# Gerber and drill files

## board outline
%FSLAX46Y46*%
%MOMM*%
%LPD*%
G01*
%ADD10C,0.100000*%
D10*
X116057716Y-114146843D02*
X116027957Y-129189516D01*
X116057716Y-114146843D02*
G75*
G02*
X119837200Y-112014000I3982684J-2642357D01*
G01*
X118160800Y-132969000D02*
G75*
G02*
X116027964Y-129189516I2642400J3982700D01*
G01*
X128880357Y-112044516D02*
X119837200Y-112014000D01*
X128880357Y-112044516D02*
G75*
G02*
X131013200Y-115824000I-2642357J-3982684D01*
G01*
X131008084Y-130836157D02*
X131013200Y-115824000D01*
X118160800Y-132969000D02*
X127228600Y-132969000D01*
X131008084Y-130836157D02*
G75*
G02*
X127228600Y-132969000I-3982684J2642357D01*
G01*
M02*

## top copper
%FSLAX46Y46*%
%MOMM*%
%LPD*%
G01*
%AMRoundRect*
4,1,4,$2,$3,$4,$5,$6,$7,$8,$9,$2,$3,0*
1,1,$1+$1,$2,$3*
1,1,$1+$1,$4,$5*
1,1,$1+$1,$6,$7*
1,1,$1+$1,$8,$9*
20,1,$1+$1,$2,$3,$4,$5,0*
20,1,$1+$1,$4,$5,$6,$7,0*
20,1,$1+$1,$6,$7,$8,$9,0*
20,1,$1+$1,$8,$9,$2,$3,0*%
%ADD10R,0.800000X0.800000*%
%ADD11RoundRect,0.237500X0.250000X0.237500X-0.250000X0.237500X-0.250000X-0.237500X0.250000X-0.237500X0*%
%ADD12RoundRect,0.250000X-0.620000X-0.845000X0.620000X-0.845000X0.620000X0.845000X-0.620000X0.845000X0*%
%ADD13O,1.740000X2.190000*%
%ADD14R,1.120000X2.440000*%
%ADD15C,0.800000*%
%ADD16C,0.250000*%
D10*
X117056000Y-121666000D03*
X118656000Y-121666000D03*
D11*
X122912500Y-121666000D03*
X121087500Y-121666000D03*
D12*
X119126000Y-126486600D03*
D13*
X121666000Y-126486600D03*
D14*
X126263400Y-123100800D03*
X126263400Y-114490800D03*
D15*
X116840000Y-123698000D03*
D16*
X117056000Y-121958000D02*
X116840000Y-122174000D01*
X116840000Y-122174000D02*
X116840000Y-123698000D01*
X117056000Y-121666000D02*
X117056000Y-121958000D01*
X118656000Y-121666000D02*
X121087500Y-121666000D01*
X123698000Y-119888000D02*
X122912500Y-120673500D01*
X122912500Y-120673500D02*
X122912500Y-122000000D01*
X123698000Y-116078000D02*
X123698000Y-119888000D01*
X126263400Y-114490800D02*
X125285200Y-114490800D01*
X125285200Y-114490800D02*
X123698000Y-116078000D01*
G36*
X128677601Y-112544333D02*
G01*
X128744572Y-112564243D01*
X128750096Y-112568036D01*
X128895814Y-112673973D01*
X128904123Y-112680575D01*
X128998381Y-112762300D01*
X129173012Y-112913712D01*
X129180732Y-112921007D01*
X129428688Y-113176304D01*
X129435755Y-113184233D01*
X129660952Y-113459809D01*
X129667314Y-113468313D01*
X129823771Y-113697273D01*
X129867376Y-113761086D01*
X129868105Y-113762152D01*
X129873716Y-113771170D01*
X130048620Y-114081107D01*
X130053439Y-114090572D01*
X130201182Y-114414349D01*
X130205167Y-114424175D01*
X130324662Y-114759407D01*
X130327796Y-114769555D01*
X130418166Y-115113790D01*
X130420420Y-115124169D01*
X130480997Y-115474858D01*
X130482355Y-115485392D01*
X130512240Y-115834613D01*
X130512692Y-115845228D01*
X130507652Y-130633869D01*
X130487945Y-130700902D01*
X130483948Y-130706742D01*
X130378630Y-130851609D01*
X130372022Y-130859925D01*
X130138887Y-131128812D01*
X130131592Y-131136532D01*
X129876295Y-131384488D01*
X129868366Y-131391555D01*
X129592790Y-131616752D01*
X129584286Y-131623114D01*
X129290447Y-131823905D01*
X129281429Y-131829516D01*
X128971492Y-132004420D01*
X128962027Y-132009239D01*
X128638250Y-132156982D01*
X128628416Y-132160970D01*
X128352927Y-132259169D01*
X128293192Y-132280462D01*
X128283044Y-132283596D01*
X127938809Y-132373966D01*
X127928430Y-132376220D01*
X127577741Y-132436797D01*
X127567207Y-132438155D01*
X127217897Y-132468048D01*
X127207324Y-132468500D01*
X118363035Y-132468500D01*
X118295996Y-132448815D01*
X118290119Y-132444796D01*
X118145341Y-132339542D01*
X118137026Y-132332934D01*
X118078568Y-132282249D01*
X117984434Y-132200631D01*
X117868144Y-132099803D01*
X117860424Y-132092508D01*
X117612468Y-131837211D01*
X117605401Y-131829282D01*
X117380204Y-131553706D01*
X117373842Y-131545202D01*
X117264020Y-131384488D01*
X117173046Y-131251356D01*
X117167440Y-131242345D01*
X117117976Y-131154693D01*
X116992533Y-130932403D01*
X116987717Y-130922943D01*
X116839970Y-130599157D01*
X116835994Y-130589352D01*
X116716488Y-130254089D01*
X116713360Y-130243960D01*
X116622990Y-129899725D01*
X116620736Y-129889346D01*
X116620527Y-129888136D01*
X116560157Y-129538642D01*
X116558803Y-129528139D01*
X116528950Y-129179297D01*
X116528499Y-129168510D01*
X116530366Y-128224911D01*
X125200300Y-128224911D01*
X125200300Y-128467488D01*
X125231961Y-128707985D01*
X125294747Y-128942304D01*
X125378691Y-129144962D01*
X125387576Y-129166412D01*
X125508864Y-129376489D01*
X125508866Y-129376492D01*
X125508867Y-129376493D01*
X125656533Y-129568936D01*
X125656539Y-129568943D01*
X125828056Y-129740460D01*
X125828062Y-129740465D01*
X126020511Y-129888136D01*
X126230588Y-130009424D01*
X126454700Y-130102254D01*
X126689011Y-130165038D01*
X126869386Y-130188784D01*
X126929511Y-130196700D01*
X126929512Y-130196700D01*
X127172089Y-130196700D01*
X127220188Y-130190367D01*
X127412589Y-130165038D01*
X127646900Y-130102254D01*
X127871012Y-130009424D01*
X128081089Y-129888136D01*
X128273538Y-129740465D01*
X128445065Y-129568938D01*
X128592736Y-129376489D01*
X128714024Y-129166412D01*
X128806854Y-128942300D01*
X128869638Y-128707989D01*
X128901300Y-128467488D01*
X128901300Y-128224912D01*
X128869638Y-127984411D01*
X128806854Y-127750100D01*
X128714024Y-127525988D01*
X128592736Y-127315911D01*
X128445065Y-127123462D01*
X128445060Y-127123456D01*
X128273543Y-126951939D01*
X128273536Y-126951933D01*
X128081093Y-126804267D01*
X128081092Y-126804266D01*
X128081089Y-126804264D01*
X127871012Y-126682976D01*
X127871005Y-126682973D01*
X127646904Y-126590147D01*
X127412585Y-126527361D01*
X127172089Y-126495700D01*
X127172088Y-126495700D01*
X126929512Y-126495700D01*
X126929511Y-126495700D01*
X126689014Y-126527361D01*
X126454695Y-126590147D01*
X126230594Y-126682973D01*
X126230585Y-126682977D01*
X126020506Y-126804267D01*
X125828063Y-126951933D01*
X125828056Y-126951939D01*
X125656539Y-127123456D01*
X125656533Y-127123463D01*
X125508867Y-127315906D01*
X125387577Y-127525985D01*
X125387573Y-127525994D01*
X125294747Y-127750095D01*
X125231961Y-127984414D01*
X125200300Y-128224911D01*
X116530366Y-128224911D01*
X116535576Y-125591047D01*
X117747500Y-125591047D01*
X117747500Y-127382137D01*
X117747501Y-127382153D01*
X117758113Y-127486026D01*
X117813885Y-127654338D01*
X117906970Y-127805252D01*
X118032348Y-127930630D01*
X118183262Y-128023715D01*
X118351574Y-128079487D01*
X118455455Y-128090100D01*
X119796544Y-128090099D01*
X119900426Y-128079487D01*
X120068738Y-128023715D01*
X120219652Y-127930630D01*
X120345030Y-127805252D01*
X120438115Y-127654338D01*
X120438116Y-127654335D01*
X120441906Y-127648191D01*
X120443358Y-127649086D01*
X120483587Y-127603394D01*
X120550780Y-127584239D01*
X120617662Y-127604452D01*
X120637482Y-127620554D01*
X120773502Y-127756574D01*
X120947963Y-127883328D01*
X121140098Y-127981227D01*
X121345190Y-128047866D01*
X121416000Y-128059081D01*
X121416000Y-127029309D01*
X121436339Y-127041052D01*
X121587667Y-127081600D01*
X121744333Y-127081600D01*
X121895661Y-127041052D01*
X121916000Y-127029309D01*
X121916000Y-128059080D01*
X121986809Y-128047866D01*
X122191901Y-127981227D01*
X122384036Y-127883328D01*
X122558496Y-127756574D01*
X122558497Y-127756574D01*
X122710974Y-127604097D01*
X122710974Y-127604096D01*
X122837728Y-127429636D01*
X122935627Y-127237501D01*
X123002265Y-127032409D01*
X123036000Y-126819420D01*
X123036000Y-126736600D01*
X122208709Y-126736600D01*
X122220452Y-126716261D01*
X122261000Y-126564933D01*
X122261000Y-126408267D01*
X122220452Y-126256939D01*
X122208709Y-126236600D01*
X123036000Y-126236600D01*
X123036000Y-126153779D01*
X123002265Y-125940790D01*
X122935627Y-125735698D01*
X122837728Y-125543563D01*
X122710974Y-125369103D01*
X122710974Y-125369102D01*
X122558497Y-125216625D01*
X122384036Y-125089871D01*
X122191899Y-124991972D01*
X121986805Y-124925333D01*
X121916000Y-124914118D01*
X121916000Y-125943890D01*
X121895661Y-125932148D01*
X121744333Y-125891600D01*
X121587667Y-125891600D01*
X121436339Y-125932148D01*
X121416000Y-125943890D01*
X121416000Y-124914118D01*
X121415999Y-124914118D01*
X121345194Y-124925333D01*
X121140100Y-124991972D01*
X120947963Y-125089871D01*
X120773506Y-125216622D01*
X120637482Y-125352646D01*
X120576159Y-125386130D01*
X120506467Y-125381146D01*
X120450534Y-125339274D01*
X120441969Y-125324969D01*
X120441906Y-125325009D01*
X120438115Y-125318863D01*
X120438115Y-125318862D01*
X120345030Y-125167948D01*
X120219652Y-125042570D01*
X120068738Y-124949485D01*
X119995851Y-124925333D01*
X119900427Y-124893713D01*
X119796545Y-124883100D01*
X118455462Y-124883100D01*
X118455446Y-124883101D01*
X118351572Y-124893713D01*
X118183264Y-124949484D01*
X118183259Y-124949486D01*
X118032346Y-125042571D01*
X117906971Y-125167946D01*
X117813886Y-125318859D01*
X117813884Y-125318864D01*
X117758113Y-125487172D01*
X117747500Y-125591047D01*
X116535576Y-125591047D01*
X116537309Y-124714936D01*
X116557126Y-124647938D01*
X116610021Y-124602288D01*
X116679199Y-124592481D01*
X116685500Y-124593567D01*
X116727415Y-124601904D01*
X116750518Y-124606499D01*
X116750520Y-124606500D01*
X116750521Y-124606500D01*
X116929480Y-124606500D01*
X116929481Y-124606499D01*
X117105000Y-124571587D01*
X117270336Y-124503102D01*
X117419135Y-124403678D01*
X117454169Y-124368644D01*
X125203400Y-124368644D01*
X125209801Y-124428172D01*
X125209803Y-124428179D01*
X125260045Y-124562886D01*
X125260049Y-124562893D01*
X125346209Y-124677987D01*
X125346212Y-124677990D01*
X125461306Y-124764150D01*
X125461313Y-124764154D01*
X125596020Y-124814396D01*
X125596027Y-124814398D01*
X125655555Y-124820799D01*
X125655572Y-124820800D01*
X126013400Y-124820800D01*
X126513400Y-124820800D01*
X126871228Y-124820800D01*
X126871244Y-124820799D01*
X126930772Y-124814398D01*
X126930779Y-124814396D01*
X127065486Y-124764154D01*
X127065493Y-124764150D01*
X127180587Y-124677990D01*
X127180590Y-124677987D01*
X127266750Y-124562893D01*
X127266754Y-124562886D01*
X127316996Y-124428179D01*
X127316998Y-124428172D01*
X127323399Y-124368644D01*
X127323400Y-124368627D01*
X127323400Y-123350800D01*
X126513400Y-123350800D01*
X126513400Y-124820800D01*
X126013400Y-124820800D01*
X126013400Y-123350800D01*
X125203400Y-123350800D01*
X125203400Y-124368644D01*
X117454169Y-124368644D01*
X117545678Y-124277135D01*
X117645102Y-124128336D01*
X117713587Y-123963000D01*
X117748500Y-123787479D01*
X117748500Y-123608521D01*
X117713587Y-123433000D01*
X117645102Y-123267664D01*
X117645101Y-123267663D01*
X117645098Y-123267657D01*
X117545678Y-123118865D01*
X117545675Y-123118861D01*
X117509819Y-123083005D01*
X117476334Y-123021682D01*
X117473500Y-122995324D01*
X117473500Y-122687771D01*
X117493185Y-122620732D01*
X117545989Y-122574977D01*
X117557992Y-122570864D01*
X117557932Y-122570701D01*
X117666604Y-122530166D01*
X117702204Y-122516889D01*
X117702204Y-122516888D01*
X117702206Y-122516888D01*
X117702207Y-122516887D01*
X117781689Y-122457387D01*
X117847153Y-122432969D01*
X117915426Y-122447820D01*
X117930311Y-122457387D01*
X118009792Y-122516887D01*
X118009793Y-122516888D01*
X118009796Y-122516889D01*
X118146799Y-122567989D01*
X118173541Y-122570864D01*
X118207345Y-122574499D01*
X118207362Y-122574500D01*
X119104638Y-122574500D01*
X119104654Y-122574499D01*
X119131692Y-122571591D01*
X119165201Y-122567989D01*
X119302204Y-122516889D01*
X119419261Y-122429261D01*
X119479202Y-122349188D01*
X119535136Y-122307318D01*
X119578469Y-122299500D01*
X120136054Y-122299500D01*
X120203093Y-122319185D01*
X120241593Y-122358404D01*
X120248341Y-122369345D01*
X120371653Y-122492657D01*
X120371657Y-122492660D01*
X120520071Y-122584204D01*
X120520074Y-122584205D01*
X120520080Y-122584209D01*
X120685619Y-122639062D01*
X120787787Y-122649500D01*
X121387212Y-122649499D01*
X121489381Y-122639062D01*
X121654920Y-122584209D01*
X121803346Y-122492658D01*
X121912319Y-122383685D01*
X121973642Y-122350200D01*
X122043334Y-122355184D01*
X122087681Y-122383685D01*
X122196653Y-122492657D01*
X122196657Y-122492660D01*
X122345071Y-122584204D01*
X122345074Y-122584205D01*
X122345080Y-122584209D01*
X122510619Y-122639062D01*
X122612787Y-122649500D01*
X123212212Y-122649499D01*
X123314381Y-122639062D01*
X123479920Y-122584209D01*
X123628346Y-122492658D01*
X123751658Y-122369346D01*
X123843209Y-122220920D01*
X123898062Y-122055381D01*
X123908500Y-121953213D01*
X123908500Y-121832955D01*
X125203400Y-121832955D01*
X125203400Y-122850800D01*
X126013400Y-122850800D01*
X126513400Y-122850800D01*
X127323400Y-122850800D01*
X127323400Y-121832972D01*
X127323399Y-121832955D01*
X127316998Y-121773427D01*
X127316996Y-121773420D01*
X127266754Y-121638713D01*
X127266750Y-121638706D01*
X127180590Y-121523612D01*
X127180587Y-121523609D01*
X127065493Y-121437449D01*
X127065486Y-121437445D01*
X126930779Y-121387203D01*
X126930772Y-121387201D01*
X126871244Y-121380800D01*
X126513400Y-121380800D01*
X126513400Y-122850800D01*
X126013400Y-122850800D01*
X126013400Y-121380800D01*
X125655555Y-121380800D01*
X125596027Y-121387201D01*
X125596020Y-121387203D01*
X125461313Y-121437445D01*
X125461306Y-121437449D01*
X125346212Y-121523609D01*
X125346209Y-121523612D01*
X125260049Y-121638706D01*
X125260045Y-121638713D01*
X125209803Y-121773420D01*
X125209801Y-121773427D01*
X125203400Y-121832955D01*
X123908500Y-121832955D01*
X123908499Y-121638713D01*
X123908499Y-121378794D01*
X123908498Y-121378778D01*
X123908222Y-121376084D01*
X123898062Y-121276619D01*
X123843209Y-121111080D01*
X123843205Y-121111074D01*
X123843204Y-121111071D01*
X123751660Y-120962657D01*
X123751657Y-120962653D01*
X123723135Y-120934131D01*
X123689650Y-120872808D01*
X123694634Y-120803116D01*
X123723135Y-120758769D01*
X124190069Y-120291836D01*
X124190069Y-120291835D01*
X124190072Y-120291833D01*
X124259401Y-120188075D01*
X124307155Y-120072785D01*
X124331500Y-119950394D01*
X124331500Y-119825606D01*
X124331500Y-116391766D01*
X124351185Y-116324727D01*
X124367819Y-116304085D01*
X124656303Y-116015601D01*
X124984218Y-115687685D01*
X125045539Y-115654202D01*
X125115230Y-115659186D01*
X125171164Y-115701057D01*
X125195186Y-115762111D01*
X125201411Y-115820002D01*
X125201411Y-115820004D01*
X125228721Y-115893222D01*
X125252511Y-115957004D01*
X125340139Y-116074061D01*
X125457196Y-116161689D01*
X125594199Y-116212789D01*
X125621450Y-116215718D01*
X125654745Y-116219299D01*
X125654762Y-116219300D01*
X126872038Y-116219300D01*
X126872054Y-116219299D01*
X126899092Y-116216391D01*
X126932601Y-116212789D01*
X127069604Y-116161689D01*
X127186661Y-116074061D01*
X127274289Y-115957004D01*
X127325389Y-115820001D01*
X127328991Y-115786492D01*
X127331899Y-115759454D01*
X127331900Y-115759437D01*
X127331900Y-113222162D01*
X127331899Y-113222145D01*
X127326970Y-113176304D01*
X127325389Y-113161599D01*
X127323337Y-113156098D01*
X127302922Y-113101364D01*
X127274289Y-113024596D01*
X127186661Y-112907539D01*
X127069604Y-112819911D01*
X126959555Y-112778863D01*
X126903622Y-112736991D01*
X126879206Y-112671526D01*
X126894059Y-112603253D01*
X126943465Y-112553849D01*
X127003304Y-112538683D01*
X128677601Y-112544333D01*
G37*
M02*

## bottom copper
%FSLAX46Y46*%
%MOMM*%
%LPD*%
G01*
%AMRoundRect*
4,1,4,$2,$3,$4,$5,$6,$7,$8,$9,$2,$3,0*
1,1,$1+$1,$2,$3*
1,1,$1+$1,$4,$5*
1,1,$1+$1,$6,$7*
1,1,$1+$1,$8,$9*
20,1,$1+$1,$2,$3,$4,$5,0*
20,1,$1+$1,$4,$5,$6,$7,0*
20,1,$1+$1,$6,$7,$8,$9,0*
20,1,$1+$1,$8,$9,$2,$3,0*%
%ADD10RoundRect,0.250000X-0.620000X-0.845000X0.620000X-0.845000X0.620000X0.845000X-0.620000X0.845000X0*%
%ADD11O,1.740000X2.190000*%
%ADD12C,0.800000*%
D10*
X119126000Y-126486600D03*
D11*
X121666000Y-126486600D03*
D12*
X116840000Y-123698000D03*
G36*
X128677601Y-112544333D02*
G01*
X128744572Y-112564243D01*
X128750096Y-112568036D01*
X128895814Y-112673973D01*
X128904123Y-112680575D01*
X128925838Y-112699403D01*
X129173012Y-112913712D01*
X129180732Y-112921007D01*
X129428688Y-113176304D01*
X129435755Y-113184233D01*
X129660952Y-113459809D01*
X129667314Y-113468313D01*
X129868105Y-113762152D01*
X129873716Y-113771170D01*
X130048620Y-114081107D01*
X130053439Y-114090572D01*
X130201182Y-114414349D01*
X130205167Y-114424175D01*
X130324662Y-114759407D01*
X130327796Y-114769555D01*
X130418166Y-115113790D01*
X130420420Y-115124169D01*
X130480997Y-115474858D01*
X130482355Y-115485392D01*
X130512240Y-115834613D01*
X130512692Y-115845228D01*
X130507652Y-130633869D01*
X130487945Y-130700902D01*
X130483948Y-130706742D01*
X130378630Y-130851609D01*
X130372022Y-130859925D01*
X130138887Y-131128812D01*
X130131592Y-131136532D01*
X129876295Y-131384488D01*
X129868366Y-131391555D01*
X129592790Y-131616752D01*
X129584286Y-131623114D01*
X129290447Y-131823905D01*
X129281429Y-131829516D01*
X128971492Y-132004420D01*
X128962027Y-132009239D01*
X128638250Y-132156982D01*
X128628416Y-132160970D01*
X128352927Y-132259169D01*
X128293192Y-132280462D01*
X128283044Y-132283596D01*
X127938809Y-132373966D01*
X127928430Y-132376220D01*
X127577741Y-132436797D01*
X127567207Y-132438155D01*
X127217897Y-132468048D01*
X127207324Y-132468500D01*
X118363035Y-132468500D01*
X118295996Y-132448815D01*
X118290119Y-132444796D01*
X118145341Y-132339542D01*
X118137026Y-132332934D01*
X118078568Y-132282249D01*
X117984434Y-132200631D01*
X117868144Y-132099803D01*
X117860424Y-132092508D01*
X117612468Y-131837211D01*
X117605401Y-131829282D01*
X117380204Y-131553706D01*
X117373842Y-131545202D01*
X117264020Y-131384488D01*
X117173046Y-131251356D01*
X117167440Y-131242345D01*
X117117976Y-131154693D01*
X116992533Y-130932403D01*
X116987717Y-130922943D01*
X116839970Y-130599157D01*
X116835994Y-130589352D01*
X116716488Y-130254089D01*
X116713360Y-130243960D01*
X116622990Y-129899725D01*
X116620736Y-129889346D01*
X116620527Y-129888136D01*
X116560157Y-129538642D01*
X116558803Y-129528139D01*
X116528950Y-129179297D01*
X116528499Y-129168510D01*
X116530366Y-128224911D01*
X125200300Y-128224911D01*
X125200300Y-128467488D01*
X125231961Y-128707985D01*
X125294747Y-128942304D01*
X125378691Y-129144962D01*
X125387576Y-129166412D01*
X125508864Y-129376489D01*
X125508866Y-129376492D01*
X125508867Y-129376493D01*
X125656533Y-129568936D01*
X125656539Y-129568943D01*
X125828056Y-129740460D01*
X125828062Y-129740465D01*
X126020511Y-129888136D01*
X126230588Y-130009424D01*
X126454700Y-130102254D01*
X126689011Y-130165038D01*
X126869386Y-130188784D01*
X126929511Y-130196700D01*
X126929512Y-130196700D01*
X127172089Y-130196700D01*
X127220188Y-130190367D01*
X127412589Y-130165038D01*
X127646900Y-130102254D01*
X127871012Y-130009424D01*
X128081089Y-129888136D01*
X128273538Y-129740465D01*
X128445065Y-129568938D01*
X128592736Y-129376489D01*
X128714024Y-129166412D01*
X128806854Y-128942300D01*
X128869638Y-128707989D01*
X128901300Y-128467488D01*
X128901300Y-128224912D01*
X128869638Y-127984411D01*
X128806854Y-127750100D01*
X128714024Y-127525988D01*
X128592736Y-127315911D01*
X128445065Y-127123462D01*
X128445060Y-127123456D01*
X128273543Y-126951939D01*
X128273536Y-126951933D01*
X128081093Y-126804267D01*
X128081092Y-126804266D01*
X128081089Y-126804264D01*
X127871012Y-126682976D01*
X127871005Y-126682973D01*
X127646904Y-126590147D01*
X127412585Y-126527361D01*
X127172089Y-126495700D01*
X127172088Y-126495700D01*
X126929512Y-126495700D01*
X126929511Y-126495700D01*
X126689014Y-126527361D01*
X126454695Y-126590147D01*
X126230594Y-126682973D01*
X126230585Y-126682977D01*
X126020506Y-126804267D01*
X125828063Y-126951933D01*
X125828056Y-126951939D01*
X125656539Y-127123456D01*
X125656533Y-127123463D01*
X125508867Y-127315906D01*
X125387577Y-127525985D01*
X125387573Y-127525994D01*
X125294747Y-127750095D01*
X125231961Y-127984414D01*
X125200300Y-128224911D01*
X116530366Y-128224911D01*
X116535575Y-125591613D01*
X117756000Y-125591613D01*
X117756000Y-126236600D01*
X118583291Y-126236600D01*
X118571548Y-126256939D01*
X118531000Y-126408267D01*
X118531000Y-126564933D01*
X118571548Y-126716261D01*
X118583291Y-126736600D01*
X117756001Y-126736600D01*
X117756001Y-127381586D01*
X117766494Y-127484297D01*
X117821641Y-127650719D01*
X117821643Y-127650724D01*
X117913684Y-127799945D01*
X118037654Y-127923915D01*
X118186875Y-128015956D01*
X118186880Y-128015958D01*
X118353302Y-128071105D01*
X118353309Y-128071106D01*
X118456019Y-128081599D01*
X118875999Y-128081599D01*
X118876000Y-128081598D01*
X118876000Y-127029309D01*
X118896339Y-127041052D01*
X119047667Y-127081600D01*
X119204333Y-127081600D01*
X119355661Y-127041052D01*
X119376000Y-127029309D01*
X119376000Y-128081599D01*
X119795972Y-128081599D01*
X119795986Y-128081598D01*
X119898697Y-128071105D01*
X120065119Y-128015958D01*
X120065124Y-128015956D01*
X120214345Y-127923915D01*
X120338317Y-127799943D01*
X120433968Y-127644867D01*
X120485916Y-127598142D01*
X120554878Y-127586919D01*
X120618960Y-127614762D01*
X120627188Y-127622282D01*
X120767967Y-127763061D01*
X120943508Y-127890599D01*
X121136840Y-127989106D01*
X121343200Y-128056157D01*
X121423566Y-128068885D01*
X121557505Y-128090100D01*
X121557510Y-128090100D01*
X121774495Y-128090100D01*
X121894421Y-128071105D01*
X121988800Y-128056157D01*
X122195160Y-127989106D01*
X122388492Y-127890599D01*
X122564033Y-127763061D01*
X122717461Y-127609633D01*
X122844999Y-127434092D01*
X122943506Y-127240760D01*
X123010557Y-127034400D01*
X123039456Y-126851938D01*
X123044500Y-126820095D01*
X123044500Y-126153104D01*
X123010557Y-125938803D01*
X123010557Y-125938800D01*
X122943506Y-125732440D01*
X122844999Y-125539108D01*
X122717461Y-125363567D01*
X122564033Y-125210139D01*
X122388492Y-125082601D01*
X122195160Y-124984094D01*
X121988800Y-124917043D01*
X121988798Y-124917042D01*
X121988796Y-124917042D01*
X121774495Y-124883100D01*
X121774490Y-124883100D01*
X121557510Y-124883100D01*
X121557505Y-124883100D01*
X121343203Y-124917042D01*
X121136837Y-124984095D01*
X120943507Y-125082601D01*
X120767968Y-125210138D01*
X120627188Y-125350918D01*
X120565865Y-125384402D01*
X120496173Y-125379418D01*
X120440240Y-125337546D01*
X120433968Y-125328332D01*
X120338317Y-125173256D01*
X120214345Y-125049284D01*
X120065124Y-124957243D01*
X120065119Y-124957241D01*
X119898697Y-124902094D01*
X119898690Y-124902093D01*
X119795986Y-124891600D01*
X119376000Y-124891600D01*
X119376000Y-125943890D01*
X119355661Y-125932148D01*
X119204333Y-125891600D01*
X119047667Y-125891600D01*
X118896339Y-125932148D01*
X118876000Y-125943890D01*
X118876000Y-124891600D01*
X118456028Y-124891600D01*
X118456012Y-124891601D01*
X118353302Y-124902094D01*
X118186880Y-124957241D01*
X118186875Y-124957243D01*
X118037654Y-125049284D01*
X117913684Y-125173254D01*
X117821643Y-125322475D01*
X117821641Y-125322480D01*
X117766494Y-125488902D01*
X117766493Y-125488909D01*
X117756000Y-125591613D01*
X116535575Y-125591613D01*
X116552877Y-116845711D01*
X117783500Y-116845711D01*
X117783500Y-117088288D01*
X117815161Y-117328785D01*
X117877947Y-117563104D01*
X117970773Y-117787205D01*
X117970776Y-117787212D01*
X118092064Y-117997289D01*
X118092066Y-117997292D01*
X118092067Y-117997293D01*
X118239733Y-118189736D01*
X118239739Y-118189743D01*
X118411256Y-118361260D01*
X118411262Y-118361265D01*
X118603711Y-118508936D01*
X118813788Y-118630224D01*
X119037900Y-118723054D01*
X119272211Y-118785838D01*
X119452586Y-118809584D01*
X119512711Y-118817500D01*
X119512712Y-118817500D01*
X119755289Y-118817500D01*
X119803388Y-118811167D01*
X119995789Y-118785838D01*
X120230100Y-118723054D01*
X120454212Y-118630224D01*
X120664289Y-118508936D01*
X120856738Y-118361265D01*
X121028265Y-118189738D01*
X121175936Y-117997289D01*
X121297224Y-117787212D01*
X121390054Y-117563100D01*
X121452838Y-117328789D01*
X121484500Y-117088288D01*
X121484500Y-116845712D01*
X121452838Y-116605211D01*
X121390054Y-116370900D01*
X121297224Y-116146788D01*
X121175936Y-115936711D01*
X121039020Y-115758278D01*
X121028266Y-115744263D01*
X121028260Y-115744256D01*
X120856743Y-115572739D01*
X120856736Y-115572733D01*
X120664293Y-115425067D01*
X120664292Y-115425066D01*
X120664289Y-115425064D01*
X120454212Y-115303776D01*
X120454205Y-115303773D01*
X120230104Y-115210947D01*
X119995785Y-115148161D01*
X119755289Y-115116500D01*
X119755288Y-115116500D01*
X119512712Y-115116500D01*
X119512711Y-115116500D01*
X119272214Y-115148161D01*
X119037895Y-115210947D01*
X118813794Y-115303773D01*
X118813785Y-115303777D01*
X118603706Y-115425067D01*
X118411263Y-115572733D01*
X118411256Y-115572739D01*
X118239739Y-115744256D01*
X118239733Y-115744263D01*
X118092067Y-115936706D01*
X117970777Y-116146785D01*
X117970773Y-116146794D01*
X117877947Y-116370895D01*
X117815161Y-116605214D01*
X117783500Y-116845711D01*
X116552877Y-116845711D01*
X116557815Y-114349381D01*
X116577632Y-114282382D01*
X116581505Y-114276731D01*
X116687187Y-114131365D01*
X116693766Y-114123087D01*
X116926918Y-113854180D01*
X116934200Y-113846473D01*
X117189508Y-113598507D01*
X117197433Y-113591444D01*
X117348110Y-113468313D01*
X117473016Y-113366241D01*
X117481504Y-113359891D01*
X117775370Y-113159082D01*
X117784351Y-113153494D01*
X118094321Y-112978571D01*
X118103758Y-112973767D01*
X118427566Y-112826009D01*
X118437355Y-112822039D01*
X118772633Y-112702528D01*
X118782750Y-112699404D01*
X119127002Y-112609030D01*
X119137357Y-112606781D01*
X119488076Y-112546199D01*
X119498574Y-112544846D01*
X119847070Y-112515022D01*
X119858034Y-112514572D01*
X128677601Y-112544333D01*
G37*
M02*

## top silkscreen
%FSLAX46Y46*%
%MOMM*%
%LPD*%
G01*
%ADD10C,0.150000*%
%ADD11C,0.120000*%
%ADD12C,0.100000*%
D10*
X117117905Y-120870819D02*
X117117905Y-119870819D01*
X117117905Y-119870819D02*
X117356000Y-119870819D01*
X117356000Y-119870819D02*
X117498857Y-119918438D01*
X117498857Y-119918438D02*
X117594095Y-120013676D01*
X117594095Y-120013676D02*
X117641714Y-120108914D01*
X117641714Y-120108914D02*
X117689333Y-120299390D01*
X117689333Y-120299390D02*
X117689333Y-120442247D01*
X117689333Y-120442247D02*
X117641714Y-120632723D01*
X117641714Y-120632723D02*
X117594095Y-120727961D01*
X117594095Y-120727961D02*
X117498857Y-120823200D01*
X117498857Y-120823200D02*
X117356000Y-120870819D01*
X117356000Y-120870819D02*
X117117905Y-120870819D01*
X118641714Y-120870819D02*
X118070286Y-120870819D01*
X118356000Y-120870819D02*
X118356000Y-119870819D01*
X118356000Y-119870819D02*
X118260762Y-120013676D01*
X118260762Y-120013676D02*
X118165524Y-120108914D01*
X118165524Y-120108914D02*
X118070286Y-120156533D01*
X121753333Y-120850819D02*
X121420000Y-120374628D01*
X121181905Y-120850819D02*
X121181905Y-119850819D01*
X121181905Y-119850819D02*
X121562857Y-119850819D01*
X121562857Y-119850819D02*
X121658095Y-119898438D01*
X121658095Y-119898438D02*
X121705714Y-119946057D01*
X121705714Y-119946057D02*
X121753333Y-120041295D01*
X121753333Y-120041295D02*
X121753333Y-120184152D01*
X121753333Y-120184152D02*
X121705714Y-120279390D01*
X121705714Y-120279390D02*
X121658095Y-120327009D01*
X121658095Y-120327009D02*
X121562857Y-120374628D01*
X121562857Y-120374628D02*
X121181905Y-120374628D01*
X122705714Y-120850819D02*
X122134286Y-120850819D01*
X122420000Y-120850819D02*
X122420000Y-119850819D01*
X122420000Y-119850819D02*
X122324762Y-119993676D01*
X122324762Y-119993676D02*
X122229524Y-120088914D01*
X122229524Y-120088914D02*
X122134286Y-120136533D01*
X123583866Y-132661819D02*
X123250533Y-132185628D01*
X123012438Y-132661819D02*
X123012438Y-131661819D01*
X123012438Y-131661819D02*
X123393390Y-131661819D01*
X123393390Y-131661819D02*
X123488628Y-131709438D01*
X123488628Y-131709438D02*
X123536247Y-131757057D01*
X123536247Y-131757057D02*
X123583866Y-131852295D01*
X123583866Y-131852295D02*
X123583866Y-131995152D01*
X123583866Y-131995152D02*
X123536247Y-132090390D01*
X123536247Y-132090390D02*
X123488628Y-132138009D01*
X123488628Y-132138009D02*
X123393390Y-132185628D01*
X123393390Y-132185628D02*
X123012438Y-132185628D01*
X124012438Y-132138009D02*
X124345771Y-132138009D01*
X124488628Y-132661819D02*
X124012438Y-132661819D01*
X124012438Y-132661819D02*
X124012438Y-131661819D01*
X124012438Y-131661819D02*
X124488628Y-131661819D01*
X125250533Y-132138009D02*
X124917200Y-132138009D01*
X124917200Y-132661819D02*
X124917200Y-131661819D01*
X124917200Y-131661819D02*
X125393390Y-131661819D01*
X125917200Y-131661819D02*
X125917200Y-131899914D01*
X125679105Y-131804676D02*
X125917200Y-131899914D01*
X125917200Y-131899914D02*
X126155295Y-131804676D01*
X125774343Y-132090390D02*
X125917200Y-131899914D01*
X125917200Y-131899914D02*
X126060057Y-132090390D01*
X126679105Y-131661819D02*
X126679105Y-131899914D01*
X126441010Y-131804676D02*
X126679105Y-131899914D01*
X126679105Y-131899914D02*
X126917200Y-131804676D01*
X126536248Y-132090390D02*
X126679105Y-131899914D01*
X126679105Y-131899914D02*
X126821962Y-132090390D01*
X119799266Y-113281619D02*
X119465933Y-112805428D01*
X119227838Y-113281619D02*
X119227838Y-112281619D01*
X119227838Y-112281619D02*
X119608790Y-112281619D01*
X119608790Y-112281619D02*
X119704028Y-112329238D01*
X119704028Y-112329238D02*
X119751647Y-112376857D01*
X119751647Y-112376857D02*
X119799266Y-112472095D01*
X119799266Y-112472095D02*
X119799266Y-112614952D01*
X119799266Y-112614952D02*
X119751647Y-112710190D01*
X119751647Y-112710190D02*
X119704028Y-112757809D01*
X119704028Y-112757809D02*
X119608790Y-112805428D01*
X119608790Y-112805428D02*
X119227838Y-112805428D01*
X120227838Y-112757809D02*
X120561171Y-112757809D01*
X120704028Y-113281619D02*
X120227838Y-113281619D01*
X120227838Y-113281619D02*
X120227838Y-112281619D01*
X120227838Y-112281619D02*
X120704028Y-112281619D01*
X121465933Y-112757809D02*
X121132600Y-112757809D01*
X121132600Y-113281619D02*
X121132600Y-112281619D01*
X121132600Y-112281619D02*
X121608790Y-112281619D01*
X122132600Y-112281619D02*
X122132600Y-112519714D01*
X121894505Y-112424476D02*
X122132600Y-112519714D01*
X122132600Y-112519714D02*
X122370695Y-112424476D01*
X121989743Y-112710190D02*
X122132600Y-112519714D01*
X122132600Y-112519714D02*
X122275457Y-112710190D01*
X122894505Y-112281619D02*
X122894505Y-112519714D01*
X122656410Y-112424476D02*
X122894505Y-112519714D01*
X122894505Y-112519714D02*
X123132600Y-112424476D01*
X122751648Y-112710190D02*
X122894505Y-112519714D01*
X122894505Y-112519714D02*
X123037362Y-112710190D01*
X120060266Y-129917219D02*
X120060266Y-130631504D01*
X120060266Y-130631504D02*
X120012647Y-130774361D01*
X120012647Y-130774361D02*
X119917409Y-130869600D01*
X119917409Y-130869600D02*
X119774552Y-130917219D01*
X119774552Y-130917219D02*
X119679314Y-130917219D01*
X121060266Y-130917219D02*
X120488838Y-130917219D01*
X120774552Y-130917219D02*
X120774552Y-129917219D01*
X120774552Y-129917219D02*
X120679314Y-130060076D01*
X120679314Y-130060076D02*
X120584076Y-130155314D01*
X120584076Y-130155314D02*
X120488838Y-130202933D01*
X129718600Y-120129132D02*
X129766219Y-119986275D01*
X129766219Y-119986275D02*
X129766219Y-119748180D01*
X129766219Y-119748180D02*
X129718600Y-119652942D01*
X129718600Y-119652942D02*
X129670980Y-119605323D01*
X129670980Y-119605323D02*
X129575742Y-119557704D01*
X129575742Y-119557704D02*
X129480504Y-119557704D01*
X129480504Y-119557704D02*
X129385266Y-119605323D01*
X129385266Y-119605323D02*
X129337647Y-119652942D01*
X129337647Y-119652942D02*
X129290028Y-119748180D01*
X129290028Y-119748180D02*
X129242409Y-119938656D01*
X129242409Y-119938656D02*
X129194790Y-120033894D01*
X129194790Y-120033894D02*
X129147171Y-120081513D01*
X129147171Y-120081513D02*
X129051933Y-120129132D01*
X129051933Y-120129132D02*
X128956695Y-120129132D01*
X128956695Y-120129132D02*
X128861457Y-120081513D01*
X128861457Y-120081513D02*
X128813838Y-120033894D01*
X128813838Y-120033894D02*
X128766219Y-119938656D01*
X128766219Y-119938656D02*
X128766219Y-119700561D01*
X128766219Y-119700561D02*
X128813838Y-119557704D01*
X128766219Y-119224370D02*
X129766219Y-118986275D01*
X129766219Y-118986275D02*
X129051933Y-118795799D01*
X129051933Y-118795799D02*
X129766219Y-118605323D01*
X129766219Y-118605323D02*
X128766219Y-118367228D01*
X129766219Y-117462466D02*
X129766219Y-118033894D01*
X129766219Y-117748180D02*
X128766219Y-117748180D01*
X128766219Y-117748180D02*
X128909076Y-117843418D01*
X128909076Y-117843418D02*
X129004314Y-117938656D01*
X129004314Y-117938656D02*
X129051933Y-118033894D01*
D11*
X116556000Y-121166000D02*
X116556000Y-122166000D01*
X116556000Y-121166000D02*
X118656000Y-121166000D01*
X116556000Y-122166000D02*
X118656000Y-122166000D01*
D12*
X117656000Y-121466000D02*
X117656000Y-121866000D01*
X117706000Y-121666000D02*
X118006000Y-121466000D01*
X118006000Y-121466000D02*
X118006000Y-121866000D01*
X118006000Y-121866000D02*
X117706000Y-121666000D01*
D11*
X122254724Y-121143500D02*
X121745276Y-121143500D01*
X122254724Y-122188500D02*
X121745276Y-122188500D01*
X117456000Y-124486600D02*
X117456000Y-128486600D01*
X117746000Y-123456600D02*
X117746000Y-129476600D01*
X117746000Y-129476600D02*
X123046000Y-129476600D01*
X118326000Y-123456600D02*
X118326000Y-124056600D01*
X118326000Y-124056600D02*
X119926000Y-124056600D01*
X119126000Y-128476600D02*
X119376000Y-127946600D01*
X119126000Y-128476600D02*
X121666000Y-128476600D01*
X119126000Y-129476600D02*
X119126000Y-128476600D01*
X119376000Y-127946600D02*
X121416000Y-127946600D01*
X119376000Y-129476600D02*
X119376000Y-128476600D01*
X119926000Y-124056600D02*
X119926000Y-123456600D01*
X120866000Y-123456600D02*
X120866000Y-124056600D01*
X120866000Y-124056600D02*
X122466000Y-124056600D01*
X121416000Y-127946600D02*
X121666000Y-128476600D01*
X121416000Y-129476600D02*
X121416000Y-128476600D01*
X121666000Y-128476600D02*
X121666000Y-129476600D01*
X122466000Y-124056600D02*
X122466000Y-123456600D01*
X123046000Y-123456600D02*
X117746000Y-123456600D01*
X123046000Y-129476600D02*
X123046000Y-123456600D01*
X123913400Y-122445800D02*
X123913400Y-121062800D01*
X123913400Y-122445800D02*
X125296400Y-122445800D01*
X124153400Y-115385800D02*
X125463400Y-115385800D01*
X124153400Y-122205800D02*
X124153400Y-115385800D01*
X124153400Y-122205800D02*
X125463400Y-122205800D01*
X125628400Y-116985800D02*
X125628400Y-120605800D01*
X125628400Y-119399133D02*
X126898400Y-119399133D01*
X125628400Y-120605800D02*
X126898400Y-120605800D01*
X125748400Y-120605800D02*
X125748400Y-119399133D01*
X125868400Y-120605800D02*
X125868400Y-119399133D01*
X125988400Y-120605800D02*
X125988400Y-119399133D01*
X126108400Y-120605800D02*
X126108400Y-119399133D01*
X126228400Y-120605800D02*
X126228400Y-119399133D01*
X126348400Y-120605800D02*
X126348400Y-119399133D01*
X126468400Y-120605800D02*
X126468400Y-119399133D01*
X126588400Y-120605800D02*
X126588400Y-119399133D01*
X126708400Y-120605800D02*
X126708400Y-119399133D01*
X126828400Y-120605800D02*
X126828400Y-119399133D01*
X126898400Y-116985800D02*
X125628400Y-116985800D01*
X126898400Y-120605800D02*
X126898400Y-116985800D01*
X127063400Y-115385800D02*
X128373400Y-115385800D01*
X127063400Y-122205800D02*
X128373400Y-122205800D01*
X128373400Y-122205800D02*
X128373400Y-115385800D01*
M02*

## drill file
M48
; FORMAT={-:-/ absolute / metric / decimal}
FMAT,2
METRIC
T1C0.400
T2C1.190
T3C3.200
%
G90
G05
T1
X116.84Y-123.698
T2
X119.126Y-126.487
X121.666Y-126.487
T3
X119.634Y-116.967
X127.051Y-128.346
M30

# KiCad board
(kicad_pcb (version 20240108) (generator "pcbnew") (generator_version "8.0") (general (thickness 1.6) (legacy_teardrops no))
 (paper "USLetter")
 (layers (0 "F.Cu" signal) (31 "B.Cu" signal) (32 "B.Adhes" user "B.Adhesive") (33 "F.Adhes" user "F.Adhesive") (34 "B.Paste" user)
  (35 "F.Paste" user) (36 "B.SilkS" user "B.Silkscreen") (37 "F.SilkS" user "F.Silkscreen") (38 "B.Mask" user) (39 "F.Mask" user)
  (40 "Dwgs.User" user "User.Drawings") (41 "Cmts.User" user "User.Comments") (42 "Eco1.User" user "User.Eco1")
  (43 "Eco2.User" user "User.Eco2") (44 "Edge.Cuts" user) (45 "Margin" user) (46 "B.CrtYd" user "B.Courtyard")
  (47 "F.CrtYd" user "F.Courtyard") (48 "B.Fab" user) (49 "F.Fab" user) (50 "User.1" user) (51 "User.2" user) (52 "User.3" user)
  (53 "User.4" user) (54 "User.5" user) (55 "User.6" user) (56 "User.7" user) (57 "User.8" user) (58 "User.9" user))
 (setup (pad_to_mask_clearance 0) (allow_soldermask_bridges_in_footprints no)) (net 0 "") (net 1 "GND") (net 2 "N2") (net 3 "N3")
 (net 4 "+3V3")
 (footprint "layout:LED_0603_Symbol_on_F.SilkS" (layer "F.Cu") (at 117.856 121.666)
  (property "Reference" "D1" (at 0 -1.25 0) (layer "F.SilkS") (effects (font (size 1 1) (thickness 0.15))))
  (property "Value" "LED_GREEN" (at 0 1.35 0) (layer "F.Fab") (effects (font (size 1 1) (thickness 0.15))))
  (fp_line (start -1.3 -0.5) (end -1.3 0.5) (stroke (width 0.12) (type solid)) (layer "F.SilkS"))
  (fp_line (start -1.3 -0.5) (end 0.8 -0.5) (stroke (width 0.12) (type solid)) (layer "F.SilkS"))
  (fp_line (start -1.3 0.5) (end 0.8 0.5) (stroke (width 0.12) (type solid)) (layer "F.SilkS"))
  (fp_line (start -0.2 -0.2) (end -0.2 0.2) (stroke (width 0.1) (type solid)) (layer "F.SilkS"))
  (fp_line (start -0.15 0) (end 0.15 -0.2) (stroke (width 0.1) (type solid)) (layer "F.SilkS"))
  (fp_line (start 0.15 -0.2) (end 0.15 0.2) (stroke (width 0.1) (type solid)) (layer "F.SilkS"))
  (fp_line (start 0.15 0.2) (end -0.15 0) (stroke (width 0.1) (type solid)) (layer "F.SilkS"))
  (pad "1" smd rect (at -0.8 0 180) (size 0.8 0.8) (layers "F.Cu" "F.Paste" "F.Mask") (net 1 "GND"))
  (pad "2" smd rect (at 0.8 0 180) (size 0.8 0.8) (layers "F.Cu" "F.Paste" "F.Mask") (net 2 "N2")))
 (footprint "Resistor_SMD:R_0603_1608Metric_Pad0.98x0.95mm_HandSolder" (layer "F.Cu") (at 122 121.666 180)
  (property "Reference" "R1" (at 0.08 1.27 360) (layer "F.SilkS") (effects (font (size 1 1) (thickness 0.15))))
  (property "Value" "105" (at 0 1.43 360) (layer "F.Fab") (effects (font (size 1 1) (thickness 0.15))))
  (fp_line (start -0.254724 0.5225) (end 0.254724 0.5225) (stroke (width 0.12) (type solid)) (layer "F.SilkS"))
  (fp_line (start -0.254724 -0.5225) (end 0.254724 -0.5225) (stroke (width 0.12) (type solid)) (layer "F.SilkS"))
  (pad "1" smd roundrect (at -0.9125 0 180) (size 0.975 0.95) (layers "F.Cu" "F.Paste" "F.Mask") (roundrect_rratio 0.25) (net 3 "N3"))
  (pad "2" smd roundrect (at 0.9125 0 180) (size 0.975 0.95) (layers "F.Cu" "F.Paste" "F.Mask") (roundrect_rratio 0.25) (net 2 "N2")))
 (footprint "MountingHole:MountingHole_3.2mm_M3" (layer "F.Cu") (at 127.0508 128.3462)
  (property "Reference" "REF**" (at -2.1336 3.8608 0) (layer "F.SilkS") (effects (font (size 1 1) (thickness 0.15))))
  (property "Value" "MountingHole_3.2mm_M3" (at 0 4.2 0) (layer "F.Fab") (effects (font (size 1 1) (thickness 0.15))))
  (pad "" np_thru_hole circle (at 0 0) (size 3.2 3.2) (drill 3.2) (layers "*.Cu" "*.Mask")))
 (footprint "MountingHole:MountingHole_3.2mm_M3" (layer "F.Cu") (at 119.634 116.967)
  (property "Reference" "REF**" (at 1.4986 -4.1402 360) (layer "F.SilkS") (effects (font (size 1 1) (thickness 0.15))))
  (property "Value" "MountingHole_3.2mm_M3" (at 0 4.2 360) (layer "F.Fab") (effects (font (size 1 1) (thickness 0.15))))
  (pad "" np_thru_hole circle (at 0 0) (size 3.2 3.2) (drill 3.2) (layers "*.Cu" "*.Mask")))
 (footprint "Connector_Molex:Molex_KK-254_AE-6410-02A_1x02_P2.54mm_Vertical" (layer "F.Cu") (at 119.126 126.4866)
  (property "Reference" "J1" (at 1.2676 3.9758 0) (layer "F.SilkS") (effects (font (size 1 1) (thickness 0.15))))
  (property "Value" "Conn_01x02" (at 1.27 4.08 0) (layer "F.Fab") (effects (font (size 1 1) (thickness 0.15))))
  (fp_line (start -1.67 -2) (end -1.67 2) (stroke (width 0.12) (type solid)) (layer "F.SilkS"))
  (fp_line (start -1.38 -3.03) (end -1.38 2.99) (stroke (width 0.12) (type solid)) (layer "F.SilkS"))
  (fp_line (start -1.38 2.99) (end 3.92 2.99) (stroke (width 0.12) (type solid)) (layer "F.SilkS"))
  (fp_line (start -0.8 -3.03) (end -0.8 -2.43) (stroke (width 0.12) (type solid)) (layer "F.SilkS"))
  (fp_line (start -0.8 -2.43) (end 0.8 -2.43) (stroke (width 0.12) (type solid)) (layer "F.SilkS"))
  (fp_line (start 0 1.99) (end 0.25 1.46) (stroke (width 0.12) (type solid)) (layer "F.SilkS"))
  (fp_line (start 0 1.99) (end 2.54 1.99) (stroke (width 0.12) (type solid)) (layer "F.SilkS"))
  (fp_line (start 0 2.99) (end 0 1.99) (stroke (width 0.12) (type solid)) (layer "F.SilkS"))
  (fp_line (start 0.25 1.46) (end 2.29 1.46) (stroke (width 0.12) (type solid)) (layer "F.SilkS"))
  (fp_line (start 0.25 2.99) (end 0.25 1.99) (stroke (width 0.12) (type solid)) (layer "F.SilkS"))
  (fp_line (start 0.8 -2.43) (end 0.8 -3.03) (stroke (width 0.12) (type solid)) (layer "F.SilkS"))
  (fp_line (start 1.74 -3.03) (end 1.74 -2.43) (stroke (width 0.12) (type solid)) (layer "F.SilkS"))
  (fp_line (start 1.74 -2.43) (end 3.34 -2.43) (stroke (width 0.12) (type solid)) (layer "F.SilkS"))
  (fp_line (start 2.29 1.46) (end 2.54 1.99) (stroke (width 0.12) (type solid)) (layer "F.SilkS"))
  (fp_line (start 2.29 2.99) (end 2.29 1.99) (stroke (width 0.12) (type solid)) (layer "F.SilkS"))
  (fp_line (start 2.54 1.99) (end 2.54 2.99) (stroke (width 0.12) (type solid)) (layer "F.SilkS"))
  (fp_line (start 3.34 -2.43) (end 3.34 -3.03) (stroke (width 0.12) (type solid)) (layer "F.SilkS"))
  (fp_line (start 3.92 -3.03) (end -1.38 -3.03) (stroke (width 0.12) (type solid)) (layer "F.SilkS"))
  (fp_line (start 3.92 2.99) (end 3.92 -3.03) (stroke (width 0.12) (type solid)) (layer "F.SilkS"))
  (pad "1" thru_hole roundrect (at 0 0) (size 1.74 2.19) (drill 1.19) (layers "*.Cu" "*.Mask") (remove_unused_layers no)
   (roundrect_rratio 0.143678) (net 1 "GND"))
  (pad "2" thru_hole oval (at 2.54 0) (size 1.74 2.19) (drill 1.19) (layers "*.Cu" "*.Mask") (remove_unused_layers no) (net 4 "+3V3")))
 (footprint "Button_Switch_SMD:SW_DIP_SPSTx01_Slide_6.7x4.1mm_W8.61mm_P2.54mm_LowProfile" (layer "F.Cu") (at 126.2634 118.7958 90)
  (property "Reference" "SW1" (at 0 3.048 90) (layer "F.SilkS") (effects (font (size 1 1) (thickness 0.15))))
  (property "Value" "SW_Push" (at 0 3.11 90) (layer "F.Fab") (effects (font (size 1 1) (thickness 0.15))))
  (fp_line (start -3.65 -2.35) (end -2.267 -2.35) (stroke (width 0.12) (type solid)) (layer "F.SilkS"))
  (fp_line (start -3.65 -2.35) (end -3.65 -0.967) (stroke (width 0.12) (type solid)) (layer "F.SilkS"))
  (fp_line (start 3.41 -2.11) (end 3.41 -0.8) (stroke (width 0.12) (type solid)) (layer "F.SilkS"))
  (fp_line (start -3.41 -2.11) (end 3.41 -2.11) (stroke (width 0.12) (type solid)) (layer "F.SilkS"))
  (fp_line (start -3.41 -2.11) (end -3.41 -0.8) (stroke (width 0.12) (type solid)) (layer "F.SilkS"))
  (fp_line (start 1.81 -0.635) (end -1.81 -0.635) (stroke (width 0.12) (type solid)) (layer "F.SilkS"))
  (fp_line (start -0.603333 -0.635) (end -0.603333 0.635) (stroke (width 0.12) (type solid)) (layer "F.SilkS"))
  (fp_line (start -1.81 -0.635) (end -1.81 0.635) (stroke (width 0.12) (type solid)) (layer "F.SilkS"))
  (fp_line (start -1.81 -0.515) (end -0.603333 -0.515) (stroke (width 0.12) (type solid)) (layer "F.SilkS"))
  (fp_line (start -1.81 -0.395) (end -0.603333 -0.395) (stroke (width 0.12) (type solid)) (layer "F.SilkS"))
  (fp_line (start -1.81 -0.275) (end -0.603333 -0.275) (stroke (width 0.12) (type solid)) (layer "F.SilkS"))
  (fp_line (start -1.81 -0.155) (end -0.603333 -0.155) (stroke (width 0.12) (type solid)) (layer "F.SilkS"))
  (fp_line (start -1.81 -0.035) (end -0.603333 -0.035) (stroke (width 0.12) (type solid)) (layer "F.SilkS"))
  (fp_line (start -1.81 0.085) (end -0.603333 0.085) (stroke (width 0.12) (type solid)) (layer "F.SilkS"))
  (fp_line (start -1.81 0.205) (end -0.603333 0.205) (stroke (width 0.12) (type solid)) (layer "F.SilkS"))
  (fp_line (start -1.81 0.325) (end -0.603333 0.325) (stroke (width 0.12) (type solid)) (layer "F.SilkS"))
  (fp_line (start -1.81 0.445) (end -0.603333 0.445) (stroke (width 0.12) (type solid)) (layer "F.SilkS"))
  (fp_line (start -1.81 0.565) (end -0.603333 0.565) (stroke (width 0.12) (type solid)) (layer "F.SilkS"))
  (fp_line (start 1.81 0.635) (end 1.81 -0.635) (stroke (width 0.12) (type solid)) (layer "F.SilkS"))
  (fp_line (start -1.81 0.635) (end 1.81 0.635) (stroke (width 0.12) (type solid)) (layer "F.SilkS"))
  (fp_line (start 3.41 0.8) (end 3.41 2.11) (stroke (width 0.12) (type solid)) (layer "F.SilkS"))
  (fp_line (start -3.41 0.8) (end -3.41 2.11) (stroke (width 0.12) (type solid)) (layer "F.SilkS"))
  (fp_line (start -3.41 2.11) (end 3.41 2.11) (stroke (width 0.12) (type solid)) (layer "F.SilkS"))
  (pad "1" smd rect (at -4.305 0 90) (size 2.44 1.12) (layers "F.Cu" "F.Paste" "F.Mask") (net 4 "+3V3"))
  (pad "2" smd rect (at 4.305 0 90) (size 2.44 1.12) (layers "F.Cu" "F.Paste" "F.Mask") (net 3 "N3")))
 (gr_line (start 116.057716 114.146843) (end 116.027957 129.189516) (stroke (width 0.1) (type default)) (layer "Edge.Cuts"))
 (gr_arc (start 116.057716 114.146843) (mid 117.69143 112.626729) (end 119.8372 112.014) (stroke (width 0.1) (type default))
  (layer "Edge.Cuts"))
 (gr_arc (start 118.1608 132.969) (mid 116.640686 131.335286) (end 116.027957 129.189516) (stroke (width 0.1) (type default))
  (layer "Edge.Cuts"))
 (gr_line (start 128.880357 112.044516) (end 119.8372 112.014) (stroke (width 0.1) (type default)) (layer "Edge.Cuts"))
 (gr_arc (start 128.880357 112.044516) (mid 130.400471 113.67823) (end 131.0132 115.824) (stroke (width 0.1) (type default))
  (layer "Edge.Cuts"))
 (gr_line (start 131.008084 130.836157) (end 131.0132 115.824) (stroke (width 0.1) (type default)) (layer "Edge.Cuts"))
 (gr_line (start 118.1608 132.969) (end 127.2286 132.969) (stroke (width 0.1) (type default)) (layer "Edge.Cuts"))
 (gr_arc (start 131.008084 130.836157) (mid 129.37437 132.356271) (end 127.2286 132.969) (stroke (width 0.1) (type default))
  (layer "Edge.Cuts"))
 (segment (start 117.056 121.958) (end 116.84 122.174) (width 0.25) (layer "F.Cu") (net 1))
 (segment (start 116.84 122.174) (end 116.84 123.698) (width 0.25) (layer "F.Cu") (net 1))
 (segment (start 117.056 121.666) (end 117.056 121.958) (width 0.25) (layer "F.Cu") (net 1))
 (via (at 116.84 123.698) (size 0.8) (drill 0.4) (layers "F.Cu" "B.Cu") (free yes) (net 1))
 (segment (start 118.656 121.666) (end 121.0875 121.666) (width 0.25) (layer "F.Cu") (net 2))
 (segment (start 123.698 119.888) (end 122.9125 120.6735) (width 0.25) (layer "F.Cu") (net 3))
 (segment (start 122.9125 120.6735) (end 122.9125 122) (width 0.25) (layer "F.Cu") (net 3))
 (segment (start 123.698 116.078) (end 123.698 119.888) (width 0.25) (layer "F.Cu") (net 3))
 (segment (start 126.2634 114.4908) (end 125.2852 114.4908) (width 0.25) (layer "F.Cu") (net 3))
 (segment (start 125.2852 114.4908) (end 123.698 116.078) (width 0.25) (layer "F.Cu") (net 3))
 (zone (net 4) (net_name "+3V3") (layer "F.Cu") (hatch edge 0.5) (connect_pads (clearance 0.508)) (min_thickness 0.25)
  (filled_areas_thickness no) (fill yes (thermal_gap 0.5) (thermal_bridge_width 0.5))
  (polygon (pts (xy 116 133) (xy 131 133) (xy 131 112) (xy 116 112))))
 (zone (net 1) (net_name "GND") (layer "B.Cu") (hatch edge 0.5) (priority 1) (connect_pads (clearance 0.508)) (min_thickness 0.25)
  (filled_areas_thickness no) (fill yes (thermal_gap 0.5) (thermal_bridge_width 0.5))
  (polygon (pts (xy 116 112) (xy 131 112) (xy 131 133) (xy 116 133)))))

